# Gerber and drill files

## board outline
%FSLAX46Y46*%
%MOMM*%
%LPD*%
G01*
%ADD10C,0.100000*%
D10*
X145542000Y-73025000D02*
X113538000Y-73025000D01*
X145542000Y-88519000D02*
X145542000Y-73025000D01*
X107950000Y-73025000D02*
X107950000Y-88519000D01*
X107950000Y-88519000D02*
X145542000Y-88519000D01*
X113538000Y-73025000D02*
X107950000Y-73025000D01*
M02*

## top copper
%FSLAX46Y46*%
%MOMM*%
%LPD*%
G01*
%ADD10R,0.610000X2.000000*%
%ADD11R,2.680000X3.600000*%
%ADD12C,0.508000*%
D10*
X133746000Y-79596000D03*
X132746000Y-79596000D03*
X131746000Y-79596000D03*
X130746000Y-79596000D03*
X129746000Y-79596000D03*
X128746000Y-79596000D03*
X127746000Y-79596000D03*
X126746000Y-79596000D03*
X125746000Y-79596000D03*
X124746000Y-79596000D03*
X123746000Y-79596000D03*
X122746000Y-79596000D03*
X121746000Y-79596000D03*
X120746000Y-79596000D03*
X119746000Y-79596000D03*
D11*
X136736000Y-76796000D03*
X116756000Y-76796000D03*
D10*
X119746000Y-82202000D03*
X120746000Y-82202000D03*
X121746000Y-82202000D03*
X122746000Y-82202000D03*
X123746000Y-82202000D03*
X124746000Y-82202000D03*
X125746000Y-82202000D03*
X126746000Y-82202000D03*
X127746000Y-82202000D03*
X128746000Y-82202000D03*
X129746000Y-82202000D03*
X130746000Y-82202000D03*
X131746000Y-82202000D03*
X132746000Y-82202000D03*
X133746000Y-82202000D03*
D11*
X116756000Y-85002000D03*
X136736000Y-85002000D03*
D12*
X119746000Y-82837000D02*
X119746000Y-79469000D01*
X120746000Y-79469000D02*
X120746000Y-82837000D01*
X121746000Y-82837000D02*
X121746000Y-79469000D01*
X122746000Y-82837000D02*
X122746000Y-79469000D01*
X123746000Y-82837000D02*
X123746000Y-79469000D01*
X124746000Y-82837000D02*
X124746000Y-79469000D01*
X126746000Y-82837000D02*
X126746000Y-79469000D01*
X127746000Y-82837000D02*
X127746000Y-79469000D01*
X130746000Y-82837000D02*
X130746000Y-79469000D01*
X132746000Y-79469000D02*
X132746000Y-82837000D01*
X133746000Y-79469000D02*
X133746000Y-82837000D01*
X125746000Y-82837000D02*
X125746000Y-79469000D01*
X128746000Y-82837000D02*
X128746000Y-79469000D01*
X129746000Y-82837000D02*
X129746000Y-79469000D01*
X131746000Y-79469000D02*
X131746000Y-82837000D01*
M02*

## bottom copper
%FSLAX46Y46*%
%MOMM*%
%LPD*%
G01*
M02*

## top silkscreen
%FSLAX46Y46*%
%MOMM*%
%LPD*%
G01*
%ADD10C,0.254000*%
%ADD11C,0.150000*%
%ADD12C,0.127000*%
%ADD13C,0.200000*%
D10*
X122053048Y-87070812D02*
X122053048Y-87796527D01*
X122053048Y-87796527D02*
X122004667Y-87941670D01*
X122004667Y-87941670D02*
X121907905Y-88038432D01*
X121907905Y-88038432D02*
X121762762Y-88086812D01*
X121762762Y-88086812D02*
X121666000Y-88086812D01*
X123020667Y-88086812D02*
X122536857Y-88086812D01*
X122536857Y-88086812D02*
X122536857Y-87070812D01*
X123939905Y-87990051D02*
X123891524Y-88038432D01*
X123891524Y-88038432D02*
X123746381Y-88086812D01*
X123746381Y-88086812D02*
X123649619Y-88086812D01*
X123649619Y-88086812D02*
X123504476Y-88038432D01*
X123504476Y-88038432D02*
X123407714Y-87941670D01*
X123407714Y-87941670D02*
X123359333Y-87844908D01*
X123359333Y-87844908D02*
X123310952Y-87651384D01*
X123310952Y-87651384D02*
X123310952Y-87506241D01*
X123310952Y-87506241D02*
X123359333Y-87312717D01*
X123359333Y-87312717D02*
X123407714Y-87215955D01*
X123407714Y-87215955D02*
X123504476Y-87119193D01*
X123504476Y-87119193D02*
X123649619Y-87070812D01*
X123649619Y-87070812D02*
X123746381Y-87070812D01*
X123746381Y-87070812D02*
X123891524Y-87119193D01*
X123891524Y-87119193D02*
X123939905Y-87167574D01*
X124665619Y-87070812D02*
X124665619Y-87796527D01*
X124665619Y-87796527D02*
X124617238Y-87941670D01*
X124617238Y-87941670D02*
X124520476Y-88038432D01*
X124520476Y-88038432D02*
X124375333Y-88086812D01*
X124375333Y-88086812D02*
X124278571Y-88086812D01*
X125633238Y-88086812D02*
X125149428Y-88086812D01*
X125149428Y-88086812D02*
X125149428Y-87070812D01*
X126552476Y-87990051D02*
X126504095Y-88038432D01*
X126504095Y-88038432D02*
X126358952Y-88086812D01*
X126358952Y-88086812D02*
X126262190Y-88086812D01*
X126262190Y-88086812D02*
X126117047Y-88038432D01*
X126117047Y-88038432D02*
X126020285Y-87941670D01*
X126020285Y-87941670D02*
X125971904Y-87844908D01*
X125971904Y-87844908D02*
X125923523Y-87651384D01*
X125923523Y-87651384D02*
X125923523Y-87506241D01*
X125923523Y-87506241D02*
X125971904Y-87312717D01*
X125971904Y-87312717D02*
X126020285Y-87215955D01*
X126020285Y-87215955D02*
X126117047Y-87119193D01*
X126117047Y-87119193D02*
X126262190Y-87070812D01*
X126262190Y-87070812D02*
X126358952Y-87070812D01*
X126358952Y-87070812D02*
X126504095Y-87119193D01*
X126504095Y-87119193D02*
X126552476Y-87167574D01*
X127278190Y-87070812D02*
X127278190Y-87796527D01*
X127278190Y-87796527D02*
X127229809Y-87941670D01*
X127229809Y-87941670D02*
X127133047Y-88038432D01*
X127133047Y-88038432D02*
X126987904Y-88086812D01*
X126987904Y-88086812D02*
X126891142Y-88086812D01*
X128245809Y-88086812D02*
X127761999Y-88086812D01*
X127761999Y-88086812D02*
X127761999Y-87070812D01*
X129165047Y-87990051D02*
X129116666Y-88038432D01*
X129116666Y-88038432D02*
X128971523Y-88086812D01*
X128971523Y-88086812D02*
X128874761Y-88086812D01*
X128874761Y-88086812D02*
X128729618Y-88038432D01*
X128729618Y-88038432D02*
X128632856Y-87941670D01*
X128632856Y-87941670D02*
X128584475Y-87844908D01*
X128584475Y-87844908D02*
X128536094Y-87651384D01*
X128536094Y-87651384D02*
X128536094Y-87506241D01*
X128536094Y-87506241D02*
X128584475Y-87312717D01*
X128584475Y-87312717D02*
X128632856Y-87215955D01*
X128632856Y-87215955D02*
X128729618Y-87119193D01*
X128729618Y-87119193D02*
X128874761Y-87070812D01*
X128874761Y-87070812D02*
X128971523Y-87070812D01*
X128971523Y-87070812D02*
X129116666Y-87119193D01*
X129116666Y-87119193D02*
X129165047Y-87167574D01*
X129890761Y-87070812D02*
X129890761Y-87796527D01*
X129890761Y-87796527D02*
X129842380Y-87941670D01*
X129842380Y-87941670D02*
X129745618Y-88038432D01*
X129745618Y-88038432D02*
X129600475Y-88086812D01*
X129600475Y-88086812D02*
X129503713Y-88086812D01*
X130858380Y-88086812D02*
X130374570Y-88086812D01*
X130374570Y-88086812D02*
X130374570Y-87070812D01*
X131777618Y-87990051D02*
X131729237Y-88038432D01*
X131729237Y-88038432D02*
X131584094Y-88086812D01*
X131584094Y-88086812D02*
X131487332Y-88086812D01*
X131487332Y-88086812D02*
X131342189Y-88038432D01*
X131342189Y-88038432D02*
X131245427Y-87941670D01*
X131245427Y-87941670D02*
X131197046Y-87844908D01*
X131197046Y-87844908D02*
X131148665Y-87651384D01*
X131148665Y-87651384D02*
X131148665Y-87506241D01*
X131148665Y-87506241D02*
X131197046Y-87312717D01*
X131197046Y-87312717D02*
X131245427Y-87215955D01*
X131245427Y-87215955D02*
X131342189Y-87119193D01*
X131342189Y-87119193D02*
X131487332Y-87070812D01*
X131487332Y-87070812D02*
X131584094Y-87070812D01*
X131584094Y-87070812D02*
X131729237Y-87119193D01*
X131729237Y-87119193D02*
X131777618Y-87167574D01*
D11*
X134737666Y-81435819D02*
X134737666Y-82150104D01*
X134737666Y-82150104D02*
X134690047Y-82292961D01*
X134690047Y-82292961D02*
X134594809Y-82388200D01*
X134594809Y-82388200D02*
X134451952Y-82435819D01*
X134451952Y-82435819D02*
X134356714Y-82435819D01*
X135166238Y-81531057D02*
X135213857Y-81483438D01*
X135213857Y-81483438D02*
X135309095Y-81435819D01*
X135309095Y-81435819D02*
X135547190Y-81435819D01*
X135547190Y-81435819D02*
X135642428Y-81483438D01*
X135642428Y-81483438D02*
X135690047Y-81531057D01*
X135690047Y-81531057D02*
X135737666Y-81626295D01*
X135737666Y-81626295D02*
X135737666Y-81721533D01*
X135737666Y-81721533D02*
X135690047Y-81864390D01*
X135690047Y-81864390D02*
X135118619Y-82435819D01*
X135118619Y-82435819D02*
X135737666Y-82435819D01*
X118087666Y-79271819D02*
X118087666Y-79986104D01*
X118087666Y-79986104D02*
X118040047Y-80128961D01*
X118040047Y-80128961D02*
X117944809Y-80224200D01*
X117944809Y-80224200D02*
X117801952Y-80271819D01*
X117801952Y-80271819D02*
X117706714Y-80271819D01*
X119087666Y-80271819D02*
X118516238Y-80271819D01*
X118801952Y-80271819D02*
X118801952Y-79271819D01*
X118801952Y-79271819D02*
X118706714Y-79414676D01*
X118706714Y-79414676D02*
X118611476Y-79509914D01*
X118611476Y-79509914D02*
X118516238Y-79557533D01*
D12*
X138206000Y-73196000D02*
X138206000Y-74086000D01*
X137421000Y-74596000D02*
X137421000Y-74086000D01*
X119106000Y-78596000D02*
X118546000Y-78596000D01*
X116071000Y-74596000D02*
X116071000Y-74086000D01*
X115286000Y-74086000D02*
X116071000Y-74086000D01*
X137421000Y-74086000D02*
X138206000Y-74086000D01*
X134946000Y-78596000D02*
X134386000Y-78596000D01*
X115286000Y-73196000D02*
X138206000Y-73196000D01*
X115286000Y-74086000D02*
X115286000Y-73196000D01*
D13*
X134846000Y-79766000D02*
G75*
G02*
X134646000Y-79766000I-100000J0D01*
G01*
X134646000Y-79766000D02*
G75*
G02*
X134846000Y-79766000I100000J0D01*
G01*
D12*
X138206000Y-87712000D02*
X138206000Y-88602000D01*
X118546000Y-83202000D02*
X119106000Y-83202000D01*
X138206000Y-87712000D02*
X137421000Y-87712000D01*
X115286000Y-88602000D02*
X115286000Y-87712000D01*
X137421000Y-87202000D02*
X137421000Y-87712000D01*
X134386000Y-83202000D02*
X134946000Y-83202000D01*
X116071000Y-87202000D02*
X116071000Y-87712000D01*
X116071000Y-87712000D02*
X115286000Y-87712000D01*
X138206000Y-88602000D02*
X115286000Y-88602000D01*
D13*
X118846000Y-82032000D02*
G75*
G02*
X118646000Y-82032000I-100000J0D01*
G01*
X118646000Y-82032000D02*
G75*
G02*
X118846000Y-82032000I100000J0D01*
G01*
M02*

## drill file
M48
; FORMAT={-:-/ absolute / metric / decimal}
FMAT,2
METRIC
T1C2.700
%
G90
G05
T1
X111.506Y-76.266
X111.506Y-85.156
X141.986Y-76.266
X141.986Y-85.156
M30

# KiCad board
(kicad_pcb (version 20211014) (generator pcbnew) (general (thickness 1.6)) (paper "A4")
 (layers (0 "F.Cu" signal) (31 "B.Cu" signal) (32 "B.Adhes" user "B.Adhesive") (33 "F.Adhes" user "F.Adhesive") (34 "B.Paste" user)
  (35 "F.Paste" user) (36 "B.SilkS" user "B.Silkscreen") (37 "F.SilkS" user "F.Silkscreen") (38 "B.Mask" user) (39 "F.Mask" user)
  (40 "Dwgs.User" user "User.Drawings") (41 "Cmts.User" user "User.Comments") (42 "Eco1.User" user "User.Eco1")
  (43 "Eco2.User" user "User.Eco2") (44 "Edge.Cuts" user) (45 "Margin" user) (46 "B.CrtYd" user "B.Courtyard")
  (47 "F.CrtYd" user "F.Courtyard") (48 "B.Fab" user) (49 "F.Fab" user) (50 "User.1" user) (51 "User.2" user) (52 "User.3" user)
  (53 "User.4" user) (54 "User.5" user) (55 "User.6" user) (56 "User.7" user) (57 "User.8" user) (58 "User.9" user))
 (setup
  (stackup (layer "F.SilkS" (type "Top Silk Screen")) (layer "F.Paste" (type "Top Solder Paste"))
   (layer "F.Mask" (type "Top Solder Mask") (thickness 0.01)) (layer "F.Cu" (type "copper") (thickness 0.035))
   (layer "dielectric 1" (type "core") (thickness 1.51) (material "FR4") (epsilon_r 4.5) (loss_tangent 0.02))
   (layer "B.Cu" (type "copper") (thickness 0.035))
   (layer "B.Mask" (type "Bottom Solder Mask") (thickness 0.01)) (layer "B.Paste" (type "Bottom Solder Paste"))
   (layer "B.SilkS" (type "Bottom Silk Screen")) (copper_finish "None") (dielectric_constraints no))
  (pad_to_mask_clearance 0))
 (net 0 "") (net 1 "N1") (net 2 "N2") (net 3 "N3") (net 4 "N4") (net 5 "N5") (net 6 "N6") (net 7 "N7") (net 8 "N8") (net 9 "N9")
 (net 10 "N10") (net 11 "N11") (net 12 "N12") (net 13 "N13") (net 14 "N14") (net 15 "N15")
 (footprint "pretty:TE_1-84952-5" (layer "F.Cu") (at 126.746 79.596 180)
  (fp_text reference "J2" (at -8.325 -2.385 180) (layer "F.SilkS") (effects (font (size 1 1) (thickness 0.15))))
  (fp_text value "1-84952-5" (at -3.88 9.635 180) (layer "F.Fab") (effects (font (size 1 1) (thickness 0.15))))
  (fp_line (start -11.46 6.4) (end -11.46 5.51) (layer "F.SilkS") (width 0.127))
  (fp_line (start -10.675 5) (end -10.675 5.51) (layer "F.SilkS") (width 0.127))
  (fp_line (start 7.64 1) (end 8.2 1) (layer "F.SilkS") (width 0.127))
  (fp_line (start 10.675 5) (end 10.675 5.51) (layer "F.SilkS") (width 0.127))
  (fp_line (start 11.46 5.51) (end 10.675 5.51) (layer "F.SilkS") (width 0.127))
  (fp_line (start -10.675 5.51) (end -11.46 5.51) (layer "F.SilkS") (width 0.127))
  (fp_line (start -8.2 1) (end -7.64 1) (layer "F.SilkS") (width 0.127))
  (fp_line (start 11.46 6.4) (end -11.46 6.4) (layer "F.SilkS") (width 0.127))
  (fp_line (start 11.46 5.51) (end 11.46 6.4) (layer "F.SilkS") (width 0.127))
  (fp_circle (center -8 -0.17) (end -7.9 -0.17) (layer "F.SilkS") (width 0.2) (fill none))
  (pad "1" smd rect locked (at -7 0 180) (size 0.61 2) (layers "F.Cu" "F.Paste" "F.Mask") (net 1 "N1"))
  (pad "2" smd rect locked (at -6 0 180) (size 0.61 2) (layers "F.Cu" "F.Paste" "F.Mask") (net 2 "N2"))
  (pad "3" smd rect locked (at -5 0 180) (size 0.61 2) (layers "F.Cu" "F.Paste" "F.Mask") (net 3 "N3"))
  (pad "4" smd rect locked (at -4 0 180) (size 0.61 2) (layers "F.Cu" "F.Paste" "F.Mask") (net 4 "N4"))
  (pad "5" smd rect locked (at -3 0 180) (size 0.61 2) (layers "F.Cu" "F.Paste" "F.Mask") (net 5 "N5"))
  (pad "6" smd rect locked (at -2 0 180) (size 0.61 2) (layers "F.Cu" "F.Paste" "F.Mask") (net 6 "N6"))
  (pad "7" smd rect locked (at -1 0 180) (size 0.61 2) (layers "F.Cu" "F.Paste" "F.Mask") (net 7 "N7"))
  (pad "8" smd rect locked (at 0 0 180) (size 0.61 2) (layers "F.Cu" "F.Paste" "F.Mask") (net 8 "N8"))
  (pad "9" smd rect locked (at 1 0 180) (size 0.61 2) (layers "F.Cu" "F.Paste" "F.Mask") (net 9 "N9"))
  (pad "10" smd rect locked (at 2 0 180) (size 0.61 2) (layers "F.Cu" "F.Paste" "F.Mask") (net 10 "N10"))
  (pad "11" smd rect locked (at 3 0 180) (size 0.61 2) (layers "F.Cu" "F.Paste" "F.Mask") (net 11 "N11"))
  (pad "12" smd rect locked (at 4 0 180) (size 0.61 2) (layers "F.Cu" "F.Paste" "F.Mask") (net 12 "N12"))
  (pad "13" smd rect locked (at 5 0 180) (size 0.61 2) (layers "F.Cu" "F.Paste" "F.Mask") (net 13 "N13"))
  (pad "14" smd rect locked (at 6 0 180) (size 0.61 2) (layers "F.Cu" "F.Paste" "F.Mask") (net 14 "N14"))
  (pad "15" smd rect locked (at 7 0 180) (size 0.61 2) (layers "F.Cu" "F.Paste" "F.Mask") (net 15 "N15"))
  (pad "S1" smd rect locked (at -9.99 2.8 180) (size 2.68 3.6) (layers "F.Cu" "F.Paste" "F.Mask"))
  (pad "S2" smd rect locked (at 9.99 2.8 180) (size 2.68 3.6) (layers "F.Cu" "F.Paste" "F.Mask")))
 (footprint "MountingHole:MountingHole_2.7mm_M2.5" (layer "F.Cu") (at 111.506 85.156)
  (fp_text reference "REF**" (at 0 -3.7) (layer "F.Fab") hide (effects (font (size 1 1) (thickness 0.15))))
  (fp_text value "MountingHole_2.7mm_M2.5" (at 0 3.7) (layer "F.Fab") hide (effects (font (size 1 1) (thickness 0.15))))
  (pad "" np_thru_hole circle locked (at 0 0) (size 2.7 2.7) (drill 2.7) (layers *.Cu *.Mask)))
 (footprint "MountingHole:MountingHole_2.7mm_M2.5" (layer "F.Cu") (at 141.986 76.266)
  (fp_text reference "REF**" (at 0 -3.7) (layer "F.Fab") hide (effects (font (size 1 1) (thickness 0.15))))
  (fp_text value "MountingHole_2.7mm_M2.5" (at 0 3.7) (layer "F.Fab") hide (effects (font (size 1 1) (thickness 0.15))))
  (pad "" np_thru_hole circle locked (at 0 0) (size 2.7 2.7) (drill 2.7) (layers *.Cu *.Mask)))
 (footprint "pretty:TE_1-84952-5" (layer "F.Cu") (at 126.746 82.202)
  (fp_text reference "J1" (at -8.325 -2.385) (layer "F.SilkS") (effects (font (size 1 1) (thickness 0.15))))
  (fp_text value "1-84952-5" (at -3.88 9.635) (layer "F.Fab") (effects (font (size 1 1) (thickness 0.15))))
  (fp_line (start 11.46 5.51) (end 11.46 6.4) (layer "F.SilkS") (width 0.127))
  (fp_line (start -8.2 1) (end -7.64 1) (layer "F.SilkS") (width 0.127))
  (fp_line (start 11.46 5.51) (end 10.675 5.51) (layer "F.SilkS") (width 0.127))
  (fp_line (start -11.46 6.4) (end -11.46 5.51) (layer "F.SilkS") (width 0.127))
  (fp_line (start 10.675 5) (end 10.675 5.51) (layer "F.SilkS") (width 0.127))
  (fp_line (start 7.64 1) (end 8.2 1) (layer "F.SilkS") (width 0.127))
  (fp_line (start -10.675 5) (end -10.675 5.51) (layer "F.SilkS") (width 0.127))
  (fp_line (start -10.675 5.51) (end -11.46 5.51) (layer "F.SilkS") (width 0.127))
  (fp_line (start 11.46 6.4) (end -11.46 6.4) (layer "F.SilkS") (width 0.127))
  (fp_circle (center -8 -0.17) (end -7.9 -0.17) (layer "F.SilkS") (width 0.2) (fill none))
  (pad "1" smd rect locked (at -7 0) (size 0.61 2) (layers "F.Cu" "F.Paste" "F.Mask") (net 15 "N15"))
  (pad "2" smd rect locked (at -6 0) (size 0.61 2) (layers "F.Cu" "F.Paste" "F.Mask") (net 14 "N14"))
  (pad "3" smd rect locked (at -5 0) (size 0.61 2) (layers "F.Cu" "F.Paste" "F.Mask") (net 13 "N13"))
  (pad "4" smd rect locked (at -4 0) (size 0.61 2) (layers "F.Cu" "F.Paste" "F.Mask") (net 12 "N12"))
  (pad "5" smd rect locked (at -3 0) (size 0.61 2) (layers "F.Cu" "F.Paste" "F.Mask") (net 11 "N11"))
  (pad "6" smd rect locked (at -2 0) (size 0.61 2) (layers "F.Cu" "F.Paste" "F.Mask") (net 10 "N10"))
  (pad "7" smd rect locked (at -1 0) (size 0.61 2) (layers "F.Cu" "F.Paste" "F.Mask") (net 9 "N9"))
  (pad "8" smd rect locked (at 0 0) (size 0.61 2) (layers "F.Cu" "F.Paste" "F.Mask") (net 8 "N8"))
  (pad "9" smd rect locked (at 1 0) (size 0.61 2) (layers "F.Cu" "F.Paste" "F.Mask") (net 7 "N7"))
  (pad "10" smd rect locked (at 2 0) (size 0.61 2) (layers "F.Cu" "F.Paste" "F.Mask") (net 6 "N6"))
  (pad "11" smd rect locked (at 3 0) (size 0.61 2) (layers "F.Cu" "F.Paste" "F.Mask") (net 5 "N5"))
  (pad "12" smd rect locked (at 4 0) (size 0.61 2) (layers "F.Cu" "F.Paste" "F.Mask") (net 4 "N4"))
  (pad "13" smd rect locked (at 5 0) (size 0.61 2) (layers "F.Cu" "F.Paste" "F.Mask") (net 3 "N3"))
  (pad "14" smd rect locked (at 6 0) (size 0.61 2) (layers "F.Cu" "F.Paste" "F.Mask") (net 2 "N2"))
  (pad "15" smd rect locked (at 7 0) (size 0.61 2) (layers "F.Cu" "F.Paste" "F.Mask") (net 1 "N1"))
  (pad "S1" smd rect locked (at -9.99 2.8) (size 2.68 3.6) (layers "F.Cu" "F.Paste" "F.Mask"))
  (pad "S2" smd rect locked (at 9.99 2.8) (size 2.68 3.6) (layers "F.Cu" "F.Paste" "F.Mask")))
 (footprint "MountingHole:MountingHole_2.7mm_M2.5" (layer "F.Cu") (at 141.986 85.156)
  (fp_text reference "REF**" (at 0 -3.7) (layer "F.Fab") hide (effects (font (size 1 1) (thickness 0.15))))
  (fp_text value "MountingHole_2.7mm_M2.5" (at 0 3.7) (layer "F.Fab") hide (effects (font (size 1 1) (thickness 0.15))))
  (pad "" np_thru_hole circle locked (at 0 0) (size 2.7 2.7) (drill 2.7) (layers *.Cu *.Mask)))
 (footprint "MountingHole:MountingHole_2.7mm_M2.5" (layer "F.Cu") (at 111.506 76.266)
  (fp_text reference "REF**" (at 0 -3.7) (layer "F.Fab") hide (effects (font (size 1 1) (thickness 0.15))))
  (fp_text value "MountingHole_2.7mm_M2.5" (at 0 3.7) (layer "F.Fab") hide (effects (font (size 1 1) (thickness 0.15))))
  (pad "" np_thru_hole circle locked (at 0 0) (size 2.7 2.7) (drill 2.7) (layers *.Cu *.Mask)))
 (gr_line (start 145.542 73.025) (end 113.538 73.025) (layer "Edge.Cuts") (width 0.1))
 (gr_line (start 145.542 88.519) (end 145.542 73.025) (layer "Edge.Cuts") (width 0.1))
 (gr_line (start 107.95 73.025) (end 107.95 88.519) (layer "Edge.Cuts") (width 0.1))
 (gr_line (start 107.95 88.519) (end 145.542 88.519) (layer "Edge.Cuts") (width 0.1))
 (gr_line (start 113.538 73.025) (end 107.95 73.025) (layer "Edge.Cuts") (width 0.1))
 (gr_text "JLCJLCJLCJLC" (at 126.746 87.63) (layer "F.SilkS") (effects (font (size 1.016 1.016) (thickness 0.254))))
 (segment (start 119.746 82.837) (end 119.746 79.469) (width 0.508) (layer "F.Cu") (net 15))
 (segment (start 120.746 79.469) (end 120.746 82.837) (width 0.508) (layer "F.Cu") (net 14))
 (segment (start 121.746 82.837) (end 121.746 79.469) (width 0.508) (layer "F.Cu") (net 13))
 (segment (start 122.746 82.837) (end 122.746 79.469) (width 0.508) (layer "F.Cu") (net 12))
 (segment (start 123.746 82.837) (end 123.746 79.469) (width 0.508) (layer "F.Cu") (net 11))
 (segment (start 124.746 82.837) (end 124.746 79.469) (width 0.508) (layer "F.Cu") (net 10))
 (segment (start 126.746 82.837) (end 126.746 79.469) (width 0.508) (layer "F.Cu") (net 8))
 (segment (start 127.746 82.837) (end 127.746 79.469) (width 0.508) (layer "F.Cu") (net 7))
 (segment (start 130.746 82.837) (end 130.746 79.469) (width 0.508) (layer "F.Cu") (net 4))
 (segment (start 132.746 79.469) (end 132.746 82.837) (width 0.508) (layer "F.Cu") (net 2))
 (segment (start 133.746 79.469) (end 133.746 82.837) (width 0.508) (layer "F.Cu") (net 1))
 (segment (start 125.746 82.837) (end 125.746 79.469) (width 0.508) (layer "F.Cu") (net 9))
 (segment (start 128.746 82.837) (end 128.746 79.469) (width 0.508) (layer "F.Cu") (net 6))
 (segment (start 129.746 82.837) (end 129.746 79.469) (width 0.508) (layer "F.Cu") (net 5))
 (segment (start 131.746 79.469) (end 131.746 82.837) (width 0.508) (layer "F.Cu") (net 3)))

